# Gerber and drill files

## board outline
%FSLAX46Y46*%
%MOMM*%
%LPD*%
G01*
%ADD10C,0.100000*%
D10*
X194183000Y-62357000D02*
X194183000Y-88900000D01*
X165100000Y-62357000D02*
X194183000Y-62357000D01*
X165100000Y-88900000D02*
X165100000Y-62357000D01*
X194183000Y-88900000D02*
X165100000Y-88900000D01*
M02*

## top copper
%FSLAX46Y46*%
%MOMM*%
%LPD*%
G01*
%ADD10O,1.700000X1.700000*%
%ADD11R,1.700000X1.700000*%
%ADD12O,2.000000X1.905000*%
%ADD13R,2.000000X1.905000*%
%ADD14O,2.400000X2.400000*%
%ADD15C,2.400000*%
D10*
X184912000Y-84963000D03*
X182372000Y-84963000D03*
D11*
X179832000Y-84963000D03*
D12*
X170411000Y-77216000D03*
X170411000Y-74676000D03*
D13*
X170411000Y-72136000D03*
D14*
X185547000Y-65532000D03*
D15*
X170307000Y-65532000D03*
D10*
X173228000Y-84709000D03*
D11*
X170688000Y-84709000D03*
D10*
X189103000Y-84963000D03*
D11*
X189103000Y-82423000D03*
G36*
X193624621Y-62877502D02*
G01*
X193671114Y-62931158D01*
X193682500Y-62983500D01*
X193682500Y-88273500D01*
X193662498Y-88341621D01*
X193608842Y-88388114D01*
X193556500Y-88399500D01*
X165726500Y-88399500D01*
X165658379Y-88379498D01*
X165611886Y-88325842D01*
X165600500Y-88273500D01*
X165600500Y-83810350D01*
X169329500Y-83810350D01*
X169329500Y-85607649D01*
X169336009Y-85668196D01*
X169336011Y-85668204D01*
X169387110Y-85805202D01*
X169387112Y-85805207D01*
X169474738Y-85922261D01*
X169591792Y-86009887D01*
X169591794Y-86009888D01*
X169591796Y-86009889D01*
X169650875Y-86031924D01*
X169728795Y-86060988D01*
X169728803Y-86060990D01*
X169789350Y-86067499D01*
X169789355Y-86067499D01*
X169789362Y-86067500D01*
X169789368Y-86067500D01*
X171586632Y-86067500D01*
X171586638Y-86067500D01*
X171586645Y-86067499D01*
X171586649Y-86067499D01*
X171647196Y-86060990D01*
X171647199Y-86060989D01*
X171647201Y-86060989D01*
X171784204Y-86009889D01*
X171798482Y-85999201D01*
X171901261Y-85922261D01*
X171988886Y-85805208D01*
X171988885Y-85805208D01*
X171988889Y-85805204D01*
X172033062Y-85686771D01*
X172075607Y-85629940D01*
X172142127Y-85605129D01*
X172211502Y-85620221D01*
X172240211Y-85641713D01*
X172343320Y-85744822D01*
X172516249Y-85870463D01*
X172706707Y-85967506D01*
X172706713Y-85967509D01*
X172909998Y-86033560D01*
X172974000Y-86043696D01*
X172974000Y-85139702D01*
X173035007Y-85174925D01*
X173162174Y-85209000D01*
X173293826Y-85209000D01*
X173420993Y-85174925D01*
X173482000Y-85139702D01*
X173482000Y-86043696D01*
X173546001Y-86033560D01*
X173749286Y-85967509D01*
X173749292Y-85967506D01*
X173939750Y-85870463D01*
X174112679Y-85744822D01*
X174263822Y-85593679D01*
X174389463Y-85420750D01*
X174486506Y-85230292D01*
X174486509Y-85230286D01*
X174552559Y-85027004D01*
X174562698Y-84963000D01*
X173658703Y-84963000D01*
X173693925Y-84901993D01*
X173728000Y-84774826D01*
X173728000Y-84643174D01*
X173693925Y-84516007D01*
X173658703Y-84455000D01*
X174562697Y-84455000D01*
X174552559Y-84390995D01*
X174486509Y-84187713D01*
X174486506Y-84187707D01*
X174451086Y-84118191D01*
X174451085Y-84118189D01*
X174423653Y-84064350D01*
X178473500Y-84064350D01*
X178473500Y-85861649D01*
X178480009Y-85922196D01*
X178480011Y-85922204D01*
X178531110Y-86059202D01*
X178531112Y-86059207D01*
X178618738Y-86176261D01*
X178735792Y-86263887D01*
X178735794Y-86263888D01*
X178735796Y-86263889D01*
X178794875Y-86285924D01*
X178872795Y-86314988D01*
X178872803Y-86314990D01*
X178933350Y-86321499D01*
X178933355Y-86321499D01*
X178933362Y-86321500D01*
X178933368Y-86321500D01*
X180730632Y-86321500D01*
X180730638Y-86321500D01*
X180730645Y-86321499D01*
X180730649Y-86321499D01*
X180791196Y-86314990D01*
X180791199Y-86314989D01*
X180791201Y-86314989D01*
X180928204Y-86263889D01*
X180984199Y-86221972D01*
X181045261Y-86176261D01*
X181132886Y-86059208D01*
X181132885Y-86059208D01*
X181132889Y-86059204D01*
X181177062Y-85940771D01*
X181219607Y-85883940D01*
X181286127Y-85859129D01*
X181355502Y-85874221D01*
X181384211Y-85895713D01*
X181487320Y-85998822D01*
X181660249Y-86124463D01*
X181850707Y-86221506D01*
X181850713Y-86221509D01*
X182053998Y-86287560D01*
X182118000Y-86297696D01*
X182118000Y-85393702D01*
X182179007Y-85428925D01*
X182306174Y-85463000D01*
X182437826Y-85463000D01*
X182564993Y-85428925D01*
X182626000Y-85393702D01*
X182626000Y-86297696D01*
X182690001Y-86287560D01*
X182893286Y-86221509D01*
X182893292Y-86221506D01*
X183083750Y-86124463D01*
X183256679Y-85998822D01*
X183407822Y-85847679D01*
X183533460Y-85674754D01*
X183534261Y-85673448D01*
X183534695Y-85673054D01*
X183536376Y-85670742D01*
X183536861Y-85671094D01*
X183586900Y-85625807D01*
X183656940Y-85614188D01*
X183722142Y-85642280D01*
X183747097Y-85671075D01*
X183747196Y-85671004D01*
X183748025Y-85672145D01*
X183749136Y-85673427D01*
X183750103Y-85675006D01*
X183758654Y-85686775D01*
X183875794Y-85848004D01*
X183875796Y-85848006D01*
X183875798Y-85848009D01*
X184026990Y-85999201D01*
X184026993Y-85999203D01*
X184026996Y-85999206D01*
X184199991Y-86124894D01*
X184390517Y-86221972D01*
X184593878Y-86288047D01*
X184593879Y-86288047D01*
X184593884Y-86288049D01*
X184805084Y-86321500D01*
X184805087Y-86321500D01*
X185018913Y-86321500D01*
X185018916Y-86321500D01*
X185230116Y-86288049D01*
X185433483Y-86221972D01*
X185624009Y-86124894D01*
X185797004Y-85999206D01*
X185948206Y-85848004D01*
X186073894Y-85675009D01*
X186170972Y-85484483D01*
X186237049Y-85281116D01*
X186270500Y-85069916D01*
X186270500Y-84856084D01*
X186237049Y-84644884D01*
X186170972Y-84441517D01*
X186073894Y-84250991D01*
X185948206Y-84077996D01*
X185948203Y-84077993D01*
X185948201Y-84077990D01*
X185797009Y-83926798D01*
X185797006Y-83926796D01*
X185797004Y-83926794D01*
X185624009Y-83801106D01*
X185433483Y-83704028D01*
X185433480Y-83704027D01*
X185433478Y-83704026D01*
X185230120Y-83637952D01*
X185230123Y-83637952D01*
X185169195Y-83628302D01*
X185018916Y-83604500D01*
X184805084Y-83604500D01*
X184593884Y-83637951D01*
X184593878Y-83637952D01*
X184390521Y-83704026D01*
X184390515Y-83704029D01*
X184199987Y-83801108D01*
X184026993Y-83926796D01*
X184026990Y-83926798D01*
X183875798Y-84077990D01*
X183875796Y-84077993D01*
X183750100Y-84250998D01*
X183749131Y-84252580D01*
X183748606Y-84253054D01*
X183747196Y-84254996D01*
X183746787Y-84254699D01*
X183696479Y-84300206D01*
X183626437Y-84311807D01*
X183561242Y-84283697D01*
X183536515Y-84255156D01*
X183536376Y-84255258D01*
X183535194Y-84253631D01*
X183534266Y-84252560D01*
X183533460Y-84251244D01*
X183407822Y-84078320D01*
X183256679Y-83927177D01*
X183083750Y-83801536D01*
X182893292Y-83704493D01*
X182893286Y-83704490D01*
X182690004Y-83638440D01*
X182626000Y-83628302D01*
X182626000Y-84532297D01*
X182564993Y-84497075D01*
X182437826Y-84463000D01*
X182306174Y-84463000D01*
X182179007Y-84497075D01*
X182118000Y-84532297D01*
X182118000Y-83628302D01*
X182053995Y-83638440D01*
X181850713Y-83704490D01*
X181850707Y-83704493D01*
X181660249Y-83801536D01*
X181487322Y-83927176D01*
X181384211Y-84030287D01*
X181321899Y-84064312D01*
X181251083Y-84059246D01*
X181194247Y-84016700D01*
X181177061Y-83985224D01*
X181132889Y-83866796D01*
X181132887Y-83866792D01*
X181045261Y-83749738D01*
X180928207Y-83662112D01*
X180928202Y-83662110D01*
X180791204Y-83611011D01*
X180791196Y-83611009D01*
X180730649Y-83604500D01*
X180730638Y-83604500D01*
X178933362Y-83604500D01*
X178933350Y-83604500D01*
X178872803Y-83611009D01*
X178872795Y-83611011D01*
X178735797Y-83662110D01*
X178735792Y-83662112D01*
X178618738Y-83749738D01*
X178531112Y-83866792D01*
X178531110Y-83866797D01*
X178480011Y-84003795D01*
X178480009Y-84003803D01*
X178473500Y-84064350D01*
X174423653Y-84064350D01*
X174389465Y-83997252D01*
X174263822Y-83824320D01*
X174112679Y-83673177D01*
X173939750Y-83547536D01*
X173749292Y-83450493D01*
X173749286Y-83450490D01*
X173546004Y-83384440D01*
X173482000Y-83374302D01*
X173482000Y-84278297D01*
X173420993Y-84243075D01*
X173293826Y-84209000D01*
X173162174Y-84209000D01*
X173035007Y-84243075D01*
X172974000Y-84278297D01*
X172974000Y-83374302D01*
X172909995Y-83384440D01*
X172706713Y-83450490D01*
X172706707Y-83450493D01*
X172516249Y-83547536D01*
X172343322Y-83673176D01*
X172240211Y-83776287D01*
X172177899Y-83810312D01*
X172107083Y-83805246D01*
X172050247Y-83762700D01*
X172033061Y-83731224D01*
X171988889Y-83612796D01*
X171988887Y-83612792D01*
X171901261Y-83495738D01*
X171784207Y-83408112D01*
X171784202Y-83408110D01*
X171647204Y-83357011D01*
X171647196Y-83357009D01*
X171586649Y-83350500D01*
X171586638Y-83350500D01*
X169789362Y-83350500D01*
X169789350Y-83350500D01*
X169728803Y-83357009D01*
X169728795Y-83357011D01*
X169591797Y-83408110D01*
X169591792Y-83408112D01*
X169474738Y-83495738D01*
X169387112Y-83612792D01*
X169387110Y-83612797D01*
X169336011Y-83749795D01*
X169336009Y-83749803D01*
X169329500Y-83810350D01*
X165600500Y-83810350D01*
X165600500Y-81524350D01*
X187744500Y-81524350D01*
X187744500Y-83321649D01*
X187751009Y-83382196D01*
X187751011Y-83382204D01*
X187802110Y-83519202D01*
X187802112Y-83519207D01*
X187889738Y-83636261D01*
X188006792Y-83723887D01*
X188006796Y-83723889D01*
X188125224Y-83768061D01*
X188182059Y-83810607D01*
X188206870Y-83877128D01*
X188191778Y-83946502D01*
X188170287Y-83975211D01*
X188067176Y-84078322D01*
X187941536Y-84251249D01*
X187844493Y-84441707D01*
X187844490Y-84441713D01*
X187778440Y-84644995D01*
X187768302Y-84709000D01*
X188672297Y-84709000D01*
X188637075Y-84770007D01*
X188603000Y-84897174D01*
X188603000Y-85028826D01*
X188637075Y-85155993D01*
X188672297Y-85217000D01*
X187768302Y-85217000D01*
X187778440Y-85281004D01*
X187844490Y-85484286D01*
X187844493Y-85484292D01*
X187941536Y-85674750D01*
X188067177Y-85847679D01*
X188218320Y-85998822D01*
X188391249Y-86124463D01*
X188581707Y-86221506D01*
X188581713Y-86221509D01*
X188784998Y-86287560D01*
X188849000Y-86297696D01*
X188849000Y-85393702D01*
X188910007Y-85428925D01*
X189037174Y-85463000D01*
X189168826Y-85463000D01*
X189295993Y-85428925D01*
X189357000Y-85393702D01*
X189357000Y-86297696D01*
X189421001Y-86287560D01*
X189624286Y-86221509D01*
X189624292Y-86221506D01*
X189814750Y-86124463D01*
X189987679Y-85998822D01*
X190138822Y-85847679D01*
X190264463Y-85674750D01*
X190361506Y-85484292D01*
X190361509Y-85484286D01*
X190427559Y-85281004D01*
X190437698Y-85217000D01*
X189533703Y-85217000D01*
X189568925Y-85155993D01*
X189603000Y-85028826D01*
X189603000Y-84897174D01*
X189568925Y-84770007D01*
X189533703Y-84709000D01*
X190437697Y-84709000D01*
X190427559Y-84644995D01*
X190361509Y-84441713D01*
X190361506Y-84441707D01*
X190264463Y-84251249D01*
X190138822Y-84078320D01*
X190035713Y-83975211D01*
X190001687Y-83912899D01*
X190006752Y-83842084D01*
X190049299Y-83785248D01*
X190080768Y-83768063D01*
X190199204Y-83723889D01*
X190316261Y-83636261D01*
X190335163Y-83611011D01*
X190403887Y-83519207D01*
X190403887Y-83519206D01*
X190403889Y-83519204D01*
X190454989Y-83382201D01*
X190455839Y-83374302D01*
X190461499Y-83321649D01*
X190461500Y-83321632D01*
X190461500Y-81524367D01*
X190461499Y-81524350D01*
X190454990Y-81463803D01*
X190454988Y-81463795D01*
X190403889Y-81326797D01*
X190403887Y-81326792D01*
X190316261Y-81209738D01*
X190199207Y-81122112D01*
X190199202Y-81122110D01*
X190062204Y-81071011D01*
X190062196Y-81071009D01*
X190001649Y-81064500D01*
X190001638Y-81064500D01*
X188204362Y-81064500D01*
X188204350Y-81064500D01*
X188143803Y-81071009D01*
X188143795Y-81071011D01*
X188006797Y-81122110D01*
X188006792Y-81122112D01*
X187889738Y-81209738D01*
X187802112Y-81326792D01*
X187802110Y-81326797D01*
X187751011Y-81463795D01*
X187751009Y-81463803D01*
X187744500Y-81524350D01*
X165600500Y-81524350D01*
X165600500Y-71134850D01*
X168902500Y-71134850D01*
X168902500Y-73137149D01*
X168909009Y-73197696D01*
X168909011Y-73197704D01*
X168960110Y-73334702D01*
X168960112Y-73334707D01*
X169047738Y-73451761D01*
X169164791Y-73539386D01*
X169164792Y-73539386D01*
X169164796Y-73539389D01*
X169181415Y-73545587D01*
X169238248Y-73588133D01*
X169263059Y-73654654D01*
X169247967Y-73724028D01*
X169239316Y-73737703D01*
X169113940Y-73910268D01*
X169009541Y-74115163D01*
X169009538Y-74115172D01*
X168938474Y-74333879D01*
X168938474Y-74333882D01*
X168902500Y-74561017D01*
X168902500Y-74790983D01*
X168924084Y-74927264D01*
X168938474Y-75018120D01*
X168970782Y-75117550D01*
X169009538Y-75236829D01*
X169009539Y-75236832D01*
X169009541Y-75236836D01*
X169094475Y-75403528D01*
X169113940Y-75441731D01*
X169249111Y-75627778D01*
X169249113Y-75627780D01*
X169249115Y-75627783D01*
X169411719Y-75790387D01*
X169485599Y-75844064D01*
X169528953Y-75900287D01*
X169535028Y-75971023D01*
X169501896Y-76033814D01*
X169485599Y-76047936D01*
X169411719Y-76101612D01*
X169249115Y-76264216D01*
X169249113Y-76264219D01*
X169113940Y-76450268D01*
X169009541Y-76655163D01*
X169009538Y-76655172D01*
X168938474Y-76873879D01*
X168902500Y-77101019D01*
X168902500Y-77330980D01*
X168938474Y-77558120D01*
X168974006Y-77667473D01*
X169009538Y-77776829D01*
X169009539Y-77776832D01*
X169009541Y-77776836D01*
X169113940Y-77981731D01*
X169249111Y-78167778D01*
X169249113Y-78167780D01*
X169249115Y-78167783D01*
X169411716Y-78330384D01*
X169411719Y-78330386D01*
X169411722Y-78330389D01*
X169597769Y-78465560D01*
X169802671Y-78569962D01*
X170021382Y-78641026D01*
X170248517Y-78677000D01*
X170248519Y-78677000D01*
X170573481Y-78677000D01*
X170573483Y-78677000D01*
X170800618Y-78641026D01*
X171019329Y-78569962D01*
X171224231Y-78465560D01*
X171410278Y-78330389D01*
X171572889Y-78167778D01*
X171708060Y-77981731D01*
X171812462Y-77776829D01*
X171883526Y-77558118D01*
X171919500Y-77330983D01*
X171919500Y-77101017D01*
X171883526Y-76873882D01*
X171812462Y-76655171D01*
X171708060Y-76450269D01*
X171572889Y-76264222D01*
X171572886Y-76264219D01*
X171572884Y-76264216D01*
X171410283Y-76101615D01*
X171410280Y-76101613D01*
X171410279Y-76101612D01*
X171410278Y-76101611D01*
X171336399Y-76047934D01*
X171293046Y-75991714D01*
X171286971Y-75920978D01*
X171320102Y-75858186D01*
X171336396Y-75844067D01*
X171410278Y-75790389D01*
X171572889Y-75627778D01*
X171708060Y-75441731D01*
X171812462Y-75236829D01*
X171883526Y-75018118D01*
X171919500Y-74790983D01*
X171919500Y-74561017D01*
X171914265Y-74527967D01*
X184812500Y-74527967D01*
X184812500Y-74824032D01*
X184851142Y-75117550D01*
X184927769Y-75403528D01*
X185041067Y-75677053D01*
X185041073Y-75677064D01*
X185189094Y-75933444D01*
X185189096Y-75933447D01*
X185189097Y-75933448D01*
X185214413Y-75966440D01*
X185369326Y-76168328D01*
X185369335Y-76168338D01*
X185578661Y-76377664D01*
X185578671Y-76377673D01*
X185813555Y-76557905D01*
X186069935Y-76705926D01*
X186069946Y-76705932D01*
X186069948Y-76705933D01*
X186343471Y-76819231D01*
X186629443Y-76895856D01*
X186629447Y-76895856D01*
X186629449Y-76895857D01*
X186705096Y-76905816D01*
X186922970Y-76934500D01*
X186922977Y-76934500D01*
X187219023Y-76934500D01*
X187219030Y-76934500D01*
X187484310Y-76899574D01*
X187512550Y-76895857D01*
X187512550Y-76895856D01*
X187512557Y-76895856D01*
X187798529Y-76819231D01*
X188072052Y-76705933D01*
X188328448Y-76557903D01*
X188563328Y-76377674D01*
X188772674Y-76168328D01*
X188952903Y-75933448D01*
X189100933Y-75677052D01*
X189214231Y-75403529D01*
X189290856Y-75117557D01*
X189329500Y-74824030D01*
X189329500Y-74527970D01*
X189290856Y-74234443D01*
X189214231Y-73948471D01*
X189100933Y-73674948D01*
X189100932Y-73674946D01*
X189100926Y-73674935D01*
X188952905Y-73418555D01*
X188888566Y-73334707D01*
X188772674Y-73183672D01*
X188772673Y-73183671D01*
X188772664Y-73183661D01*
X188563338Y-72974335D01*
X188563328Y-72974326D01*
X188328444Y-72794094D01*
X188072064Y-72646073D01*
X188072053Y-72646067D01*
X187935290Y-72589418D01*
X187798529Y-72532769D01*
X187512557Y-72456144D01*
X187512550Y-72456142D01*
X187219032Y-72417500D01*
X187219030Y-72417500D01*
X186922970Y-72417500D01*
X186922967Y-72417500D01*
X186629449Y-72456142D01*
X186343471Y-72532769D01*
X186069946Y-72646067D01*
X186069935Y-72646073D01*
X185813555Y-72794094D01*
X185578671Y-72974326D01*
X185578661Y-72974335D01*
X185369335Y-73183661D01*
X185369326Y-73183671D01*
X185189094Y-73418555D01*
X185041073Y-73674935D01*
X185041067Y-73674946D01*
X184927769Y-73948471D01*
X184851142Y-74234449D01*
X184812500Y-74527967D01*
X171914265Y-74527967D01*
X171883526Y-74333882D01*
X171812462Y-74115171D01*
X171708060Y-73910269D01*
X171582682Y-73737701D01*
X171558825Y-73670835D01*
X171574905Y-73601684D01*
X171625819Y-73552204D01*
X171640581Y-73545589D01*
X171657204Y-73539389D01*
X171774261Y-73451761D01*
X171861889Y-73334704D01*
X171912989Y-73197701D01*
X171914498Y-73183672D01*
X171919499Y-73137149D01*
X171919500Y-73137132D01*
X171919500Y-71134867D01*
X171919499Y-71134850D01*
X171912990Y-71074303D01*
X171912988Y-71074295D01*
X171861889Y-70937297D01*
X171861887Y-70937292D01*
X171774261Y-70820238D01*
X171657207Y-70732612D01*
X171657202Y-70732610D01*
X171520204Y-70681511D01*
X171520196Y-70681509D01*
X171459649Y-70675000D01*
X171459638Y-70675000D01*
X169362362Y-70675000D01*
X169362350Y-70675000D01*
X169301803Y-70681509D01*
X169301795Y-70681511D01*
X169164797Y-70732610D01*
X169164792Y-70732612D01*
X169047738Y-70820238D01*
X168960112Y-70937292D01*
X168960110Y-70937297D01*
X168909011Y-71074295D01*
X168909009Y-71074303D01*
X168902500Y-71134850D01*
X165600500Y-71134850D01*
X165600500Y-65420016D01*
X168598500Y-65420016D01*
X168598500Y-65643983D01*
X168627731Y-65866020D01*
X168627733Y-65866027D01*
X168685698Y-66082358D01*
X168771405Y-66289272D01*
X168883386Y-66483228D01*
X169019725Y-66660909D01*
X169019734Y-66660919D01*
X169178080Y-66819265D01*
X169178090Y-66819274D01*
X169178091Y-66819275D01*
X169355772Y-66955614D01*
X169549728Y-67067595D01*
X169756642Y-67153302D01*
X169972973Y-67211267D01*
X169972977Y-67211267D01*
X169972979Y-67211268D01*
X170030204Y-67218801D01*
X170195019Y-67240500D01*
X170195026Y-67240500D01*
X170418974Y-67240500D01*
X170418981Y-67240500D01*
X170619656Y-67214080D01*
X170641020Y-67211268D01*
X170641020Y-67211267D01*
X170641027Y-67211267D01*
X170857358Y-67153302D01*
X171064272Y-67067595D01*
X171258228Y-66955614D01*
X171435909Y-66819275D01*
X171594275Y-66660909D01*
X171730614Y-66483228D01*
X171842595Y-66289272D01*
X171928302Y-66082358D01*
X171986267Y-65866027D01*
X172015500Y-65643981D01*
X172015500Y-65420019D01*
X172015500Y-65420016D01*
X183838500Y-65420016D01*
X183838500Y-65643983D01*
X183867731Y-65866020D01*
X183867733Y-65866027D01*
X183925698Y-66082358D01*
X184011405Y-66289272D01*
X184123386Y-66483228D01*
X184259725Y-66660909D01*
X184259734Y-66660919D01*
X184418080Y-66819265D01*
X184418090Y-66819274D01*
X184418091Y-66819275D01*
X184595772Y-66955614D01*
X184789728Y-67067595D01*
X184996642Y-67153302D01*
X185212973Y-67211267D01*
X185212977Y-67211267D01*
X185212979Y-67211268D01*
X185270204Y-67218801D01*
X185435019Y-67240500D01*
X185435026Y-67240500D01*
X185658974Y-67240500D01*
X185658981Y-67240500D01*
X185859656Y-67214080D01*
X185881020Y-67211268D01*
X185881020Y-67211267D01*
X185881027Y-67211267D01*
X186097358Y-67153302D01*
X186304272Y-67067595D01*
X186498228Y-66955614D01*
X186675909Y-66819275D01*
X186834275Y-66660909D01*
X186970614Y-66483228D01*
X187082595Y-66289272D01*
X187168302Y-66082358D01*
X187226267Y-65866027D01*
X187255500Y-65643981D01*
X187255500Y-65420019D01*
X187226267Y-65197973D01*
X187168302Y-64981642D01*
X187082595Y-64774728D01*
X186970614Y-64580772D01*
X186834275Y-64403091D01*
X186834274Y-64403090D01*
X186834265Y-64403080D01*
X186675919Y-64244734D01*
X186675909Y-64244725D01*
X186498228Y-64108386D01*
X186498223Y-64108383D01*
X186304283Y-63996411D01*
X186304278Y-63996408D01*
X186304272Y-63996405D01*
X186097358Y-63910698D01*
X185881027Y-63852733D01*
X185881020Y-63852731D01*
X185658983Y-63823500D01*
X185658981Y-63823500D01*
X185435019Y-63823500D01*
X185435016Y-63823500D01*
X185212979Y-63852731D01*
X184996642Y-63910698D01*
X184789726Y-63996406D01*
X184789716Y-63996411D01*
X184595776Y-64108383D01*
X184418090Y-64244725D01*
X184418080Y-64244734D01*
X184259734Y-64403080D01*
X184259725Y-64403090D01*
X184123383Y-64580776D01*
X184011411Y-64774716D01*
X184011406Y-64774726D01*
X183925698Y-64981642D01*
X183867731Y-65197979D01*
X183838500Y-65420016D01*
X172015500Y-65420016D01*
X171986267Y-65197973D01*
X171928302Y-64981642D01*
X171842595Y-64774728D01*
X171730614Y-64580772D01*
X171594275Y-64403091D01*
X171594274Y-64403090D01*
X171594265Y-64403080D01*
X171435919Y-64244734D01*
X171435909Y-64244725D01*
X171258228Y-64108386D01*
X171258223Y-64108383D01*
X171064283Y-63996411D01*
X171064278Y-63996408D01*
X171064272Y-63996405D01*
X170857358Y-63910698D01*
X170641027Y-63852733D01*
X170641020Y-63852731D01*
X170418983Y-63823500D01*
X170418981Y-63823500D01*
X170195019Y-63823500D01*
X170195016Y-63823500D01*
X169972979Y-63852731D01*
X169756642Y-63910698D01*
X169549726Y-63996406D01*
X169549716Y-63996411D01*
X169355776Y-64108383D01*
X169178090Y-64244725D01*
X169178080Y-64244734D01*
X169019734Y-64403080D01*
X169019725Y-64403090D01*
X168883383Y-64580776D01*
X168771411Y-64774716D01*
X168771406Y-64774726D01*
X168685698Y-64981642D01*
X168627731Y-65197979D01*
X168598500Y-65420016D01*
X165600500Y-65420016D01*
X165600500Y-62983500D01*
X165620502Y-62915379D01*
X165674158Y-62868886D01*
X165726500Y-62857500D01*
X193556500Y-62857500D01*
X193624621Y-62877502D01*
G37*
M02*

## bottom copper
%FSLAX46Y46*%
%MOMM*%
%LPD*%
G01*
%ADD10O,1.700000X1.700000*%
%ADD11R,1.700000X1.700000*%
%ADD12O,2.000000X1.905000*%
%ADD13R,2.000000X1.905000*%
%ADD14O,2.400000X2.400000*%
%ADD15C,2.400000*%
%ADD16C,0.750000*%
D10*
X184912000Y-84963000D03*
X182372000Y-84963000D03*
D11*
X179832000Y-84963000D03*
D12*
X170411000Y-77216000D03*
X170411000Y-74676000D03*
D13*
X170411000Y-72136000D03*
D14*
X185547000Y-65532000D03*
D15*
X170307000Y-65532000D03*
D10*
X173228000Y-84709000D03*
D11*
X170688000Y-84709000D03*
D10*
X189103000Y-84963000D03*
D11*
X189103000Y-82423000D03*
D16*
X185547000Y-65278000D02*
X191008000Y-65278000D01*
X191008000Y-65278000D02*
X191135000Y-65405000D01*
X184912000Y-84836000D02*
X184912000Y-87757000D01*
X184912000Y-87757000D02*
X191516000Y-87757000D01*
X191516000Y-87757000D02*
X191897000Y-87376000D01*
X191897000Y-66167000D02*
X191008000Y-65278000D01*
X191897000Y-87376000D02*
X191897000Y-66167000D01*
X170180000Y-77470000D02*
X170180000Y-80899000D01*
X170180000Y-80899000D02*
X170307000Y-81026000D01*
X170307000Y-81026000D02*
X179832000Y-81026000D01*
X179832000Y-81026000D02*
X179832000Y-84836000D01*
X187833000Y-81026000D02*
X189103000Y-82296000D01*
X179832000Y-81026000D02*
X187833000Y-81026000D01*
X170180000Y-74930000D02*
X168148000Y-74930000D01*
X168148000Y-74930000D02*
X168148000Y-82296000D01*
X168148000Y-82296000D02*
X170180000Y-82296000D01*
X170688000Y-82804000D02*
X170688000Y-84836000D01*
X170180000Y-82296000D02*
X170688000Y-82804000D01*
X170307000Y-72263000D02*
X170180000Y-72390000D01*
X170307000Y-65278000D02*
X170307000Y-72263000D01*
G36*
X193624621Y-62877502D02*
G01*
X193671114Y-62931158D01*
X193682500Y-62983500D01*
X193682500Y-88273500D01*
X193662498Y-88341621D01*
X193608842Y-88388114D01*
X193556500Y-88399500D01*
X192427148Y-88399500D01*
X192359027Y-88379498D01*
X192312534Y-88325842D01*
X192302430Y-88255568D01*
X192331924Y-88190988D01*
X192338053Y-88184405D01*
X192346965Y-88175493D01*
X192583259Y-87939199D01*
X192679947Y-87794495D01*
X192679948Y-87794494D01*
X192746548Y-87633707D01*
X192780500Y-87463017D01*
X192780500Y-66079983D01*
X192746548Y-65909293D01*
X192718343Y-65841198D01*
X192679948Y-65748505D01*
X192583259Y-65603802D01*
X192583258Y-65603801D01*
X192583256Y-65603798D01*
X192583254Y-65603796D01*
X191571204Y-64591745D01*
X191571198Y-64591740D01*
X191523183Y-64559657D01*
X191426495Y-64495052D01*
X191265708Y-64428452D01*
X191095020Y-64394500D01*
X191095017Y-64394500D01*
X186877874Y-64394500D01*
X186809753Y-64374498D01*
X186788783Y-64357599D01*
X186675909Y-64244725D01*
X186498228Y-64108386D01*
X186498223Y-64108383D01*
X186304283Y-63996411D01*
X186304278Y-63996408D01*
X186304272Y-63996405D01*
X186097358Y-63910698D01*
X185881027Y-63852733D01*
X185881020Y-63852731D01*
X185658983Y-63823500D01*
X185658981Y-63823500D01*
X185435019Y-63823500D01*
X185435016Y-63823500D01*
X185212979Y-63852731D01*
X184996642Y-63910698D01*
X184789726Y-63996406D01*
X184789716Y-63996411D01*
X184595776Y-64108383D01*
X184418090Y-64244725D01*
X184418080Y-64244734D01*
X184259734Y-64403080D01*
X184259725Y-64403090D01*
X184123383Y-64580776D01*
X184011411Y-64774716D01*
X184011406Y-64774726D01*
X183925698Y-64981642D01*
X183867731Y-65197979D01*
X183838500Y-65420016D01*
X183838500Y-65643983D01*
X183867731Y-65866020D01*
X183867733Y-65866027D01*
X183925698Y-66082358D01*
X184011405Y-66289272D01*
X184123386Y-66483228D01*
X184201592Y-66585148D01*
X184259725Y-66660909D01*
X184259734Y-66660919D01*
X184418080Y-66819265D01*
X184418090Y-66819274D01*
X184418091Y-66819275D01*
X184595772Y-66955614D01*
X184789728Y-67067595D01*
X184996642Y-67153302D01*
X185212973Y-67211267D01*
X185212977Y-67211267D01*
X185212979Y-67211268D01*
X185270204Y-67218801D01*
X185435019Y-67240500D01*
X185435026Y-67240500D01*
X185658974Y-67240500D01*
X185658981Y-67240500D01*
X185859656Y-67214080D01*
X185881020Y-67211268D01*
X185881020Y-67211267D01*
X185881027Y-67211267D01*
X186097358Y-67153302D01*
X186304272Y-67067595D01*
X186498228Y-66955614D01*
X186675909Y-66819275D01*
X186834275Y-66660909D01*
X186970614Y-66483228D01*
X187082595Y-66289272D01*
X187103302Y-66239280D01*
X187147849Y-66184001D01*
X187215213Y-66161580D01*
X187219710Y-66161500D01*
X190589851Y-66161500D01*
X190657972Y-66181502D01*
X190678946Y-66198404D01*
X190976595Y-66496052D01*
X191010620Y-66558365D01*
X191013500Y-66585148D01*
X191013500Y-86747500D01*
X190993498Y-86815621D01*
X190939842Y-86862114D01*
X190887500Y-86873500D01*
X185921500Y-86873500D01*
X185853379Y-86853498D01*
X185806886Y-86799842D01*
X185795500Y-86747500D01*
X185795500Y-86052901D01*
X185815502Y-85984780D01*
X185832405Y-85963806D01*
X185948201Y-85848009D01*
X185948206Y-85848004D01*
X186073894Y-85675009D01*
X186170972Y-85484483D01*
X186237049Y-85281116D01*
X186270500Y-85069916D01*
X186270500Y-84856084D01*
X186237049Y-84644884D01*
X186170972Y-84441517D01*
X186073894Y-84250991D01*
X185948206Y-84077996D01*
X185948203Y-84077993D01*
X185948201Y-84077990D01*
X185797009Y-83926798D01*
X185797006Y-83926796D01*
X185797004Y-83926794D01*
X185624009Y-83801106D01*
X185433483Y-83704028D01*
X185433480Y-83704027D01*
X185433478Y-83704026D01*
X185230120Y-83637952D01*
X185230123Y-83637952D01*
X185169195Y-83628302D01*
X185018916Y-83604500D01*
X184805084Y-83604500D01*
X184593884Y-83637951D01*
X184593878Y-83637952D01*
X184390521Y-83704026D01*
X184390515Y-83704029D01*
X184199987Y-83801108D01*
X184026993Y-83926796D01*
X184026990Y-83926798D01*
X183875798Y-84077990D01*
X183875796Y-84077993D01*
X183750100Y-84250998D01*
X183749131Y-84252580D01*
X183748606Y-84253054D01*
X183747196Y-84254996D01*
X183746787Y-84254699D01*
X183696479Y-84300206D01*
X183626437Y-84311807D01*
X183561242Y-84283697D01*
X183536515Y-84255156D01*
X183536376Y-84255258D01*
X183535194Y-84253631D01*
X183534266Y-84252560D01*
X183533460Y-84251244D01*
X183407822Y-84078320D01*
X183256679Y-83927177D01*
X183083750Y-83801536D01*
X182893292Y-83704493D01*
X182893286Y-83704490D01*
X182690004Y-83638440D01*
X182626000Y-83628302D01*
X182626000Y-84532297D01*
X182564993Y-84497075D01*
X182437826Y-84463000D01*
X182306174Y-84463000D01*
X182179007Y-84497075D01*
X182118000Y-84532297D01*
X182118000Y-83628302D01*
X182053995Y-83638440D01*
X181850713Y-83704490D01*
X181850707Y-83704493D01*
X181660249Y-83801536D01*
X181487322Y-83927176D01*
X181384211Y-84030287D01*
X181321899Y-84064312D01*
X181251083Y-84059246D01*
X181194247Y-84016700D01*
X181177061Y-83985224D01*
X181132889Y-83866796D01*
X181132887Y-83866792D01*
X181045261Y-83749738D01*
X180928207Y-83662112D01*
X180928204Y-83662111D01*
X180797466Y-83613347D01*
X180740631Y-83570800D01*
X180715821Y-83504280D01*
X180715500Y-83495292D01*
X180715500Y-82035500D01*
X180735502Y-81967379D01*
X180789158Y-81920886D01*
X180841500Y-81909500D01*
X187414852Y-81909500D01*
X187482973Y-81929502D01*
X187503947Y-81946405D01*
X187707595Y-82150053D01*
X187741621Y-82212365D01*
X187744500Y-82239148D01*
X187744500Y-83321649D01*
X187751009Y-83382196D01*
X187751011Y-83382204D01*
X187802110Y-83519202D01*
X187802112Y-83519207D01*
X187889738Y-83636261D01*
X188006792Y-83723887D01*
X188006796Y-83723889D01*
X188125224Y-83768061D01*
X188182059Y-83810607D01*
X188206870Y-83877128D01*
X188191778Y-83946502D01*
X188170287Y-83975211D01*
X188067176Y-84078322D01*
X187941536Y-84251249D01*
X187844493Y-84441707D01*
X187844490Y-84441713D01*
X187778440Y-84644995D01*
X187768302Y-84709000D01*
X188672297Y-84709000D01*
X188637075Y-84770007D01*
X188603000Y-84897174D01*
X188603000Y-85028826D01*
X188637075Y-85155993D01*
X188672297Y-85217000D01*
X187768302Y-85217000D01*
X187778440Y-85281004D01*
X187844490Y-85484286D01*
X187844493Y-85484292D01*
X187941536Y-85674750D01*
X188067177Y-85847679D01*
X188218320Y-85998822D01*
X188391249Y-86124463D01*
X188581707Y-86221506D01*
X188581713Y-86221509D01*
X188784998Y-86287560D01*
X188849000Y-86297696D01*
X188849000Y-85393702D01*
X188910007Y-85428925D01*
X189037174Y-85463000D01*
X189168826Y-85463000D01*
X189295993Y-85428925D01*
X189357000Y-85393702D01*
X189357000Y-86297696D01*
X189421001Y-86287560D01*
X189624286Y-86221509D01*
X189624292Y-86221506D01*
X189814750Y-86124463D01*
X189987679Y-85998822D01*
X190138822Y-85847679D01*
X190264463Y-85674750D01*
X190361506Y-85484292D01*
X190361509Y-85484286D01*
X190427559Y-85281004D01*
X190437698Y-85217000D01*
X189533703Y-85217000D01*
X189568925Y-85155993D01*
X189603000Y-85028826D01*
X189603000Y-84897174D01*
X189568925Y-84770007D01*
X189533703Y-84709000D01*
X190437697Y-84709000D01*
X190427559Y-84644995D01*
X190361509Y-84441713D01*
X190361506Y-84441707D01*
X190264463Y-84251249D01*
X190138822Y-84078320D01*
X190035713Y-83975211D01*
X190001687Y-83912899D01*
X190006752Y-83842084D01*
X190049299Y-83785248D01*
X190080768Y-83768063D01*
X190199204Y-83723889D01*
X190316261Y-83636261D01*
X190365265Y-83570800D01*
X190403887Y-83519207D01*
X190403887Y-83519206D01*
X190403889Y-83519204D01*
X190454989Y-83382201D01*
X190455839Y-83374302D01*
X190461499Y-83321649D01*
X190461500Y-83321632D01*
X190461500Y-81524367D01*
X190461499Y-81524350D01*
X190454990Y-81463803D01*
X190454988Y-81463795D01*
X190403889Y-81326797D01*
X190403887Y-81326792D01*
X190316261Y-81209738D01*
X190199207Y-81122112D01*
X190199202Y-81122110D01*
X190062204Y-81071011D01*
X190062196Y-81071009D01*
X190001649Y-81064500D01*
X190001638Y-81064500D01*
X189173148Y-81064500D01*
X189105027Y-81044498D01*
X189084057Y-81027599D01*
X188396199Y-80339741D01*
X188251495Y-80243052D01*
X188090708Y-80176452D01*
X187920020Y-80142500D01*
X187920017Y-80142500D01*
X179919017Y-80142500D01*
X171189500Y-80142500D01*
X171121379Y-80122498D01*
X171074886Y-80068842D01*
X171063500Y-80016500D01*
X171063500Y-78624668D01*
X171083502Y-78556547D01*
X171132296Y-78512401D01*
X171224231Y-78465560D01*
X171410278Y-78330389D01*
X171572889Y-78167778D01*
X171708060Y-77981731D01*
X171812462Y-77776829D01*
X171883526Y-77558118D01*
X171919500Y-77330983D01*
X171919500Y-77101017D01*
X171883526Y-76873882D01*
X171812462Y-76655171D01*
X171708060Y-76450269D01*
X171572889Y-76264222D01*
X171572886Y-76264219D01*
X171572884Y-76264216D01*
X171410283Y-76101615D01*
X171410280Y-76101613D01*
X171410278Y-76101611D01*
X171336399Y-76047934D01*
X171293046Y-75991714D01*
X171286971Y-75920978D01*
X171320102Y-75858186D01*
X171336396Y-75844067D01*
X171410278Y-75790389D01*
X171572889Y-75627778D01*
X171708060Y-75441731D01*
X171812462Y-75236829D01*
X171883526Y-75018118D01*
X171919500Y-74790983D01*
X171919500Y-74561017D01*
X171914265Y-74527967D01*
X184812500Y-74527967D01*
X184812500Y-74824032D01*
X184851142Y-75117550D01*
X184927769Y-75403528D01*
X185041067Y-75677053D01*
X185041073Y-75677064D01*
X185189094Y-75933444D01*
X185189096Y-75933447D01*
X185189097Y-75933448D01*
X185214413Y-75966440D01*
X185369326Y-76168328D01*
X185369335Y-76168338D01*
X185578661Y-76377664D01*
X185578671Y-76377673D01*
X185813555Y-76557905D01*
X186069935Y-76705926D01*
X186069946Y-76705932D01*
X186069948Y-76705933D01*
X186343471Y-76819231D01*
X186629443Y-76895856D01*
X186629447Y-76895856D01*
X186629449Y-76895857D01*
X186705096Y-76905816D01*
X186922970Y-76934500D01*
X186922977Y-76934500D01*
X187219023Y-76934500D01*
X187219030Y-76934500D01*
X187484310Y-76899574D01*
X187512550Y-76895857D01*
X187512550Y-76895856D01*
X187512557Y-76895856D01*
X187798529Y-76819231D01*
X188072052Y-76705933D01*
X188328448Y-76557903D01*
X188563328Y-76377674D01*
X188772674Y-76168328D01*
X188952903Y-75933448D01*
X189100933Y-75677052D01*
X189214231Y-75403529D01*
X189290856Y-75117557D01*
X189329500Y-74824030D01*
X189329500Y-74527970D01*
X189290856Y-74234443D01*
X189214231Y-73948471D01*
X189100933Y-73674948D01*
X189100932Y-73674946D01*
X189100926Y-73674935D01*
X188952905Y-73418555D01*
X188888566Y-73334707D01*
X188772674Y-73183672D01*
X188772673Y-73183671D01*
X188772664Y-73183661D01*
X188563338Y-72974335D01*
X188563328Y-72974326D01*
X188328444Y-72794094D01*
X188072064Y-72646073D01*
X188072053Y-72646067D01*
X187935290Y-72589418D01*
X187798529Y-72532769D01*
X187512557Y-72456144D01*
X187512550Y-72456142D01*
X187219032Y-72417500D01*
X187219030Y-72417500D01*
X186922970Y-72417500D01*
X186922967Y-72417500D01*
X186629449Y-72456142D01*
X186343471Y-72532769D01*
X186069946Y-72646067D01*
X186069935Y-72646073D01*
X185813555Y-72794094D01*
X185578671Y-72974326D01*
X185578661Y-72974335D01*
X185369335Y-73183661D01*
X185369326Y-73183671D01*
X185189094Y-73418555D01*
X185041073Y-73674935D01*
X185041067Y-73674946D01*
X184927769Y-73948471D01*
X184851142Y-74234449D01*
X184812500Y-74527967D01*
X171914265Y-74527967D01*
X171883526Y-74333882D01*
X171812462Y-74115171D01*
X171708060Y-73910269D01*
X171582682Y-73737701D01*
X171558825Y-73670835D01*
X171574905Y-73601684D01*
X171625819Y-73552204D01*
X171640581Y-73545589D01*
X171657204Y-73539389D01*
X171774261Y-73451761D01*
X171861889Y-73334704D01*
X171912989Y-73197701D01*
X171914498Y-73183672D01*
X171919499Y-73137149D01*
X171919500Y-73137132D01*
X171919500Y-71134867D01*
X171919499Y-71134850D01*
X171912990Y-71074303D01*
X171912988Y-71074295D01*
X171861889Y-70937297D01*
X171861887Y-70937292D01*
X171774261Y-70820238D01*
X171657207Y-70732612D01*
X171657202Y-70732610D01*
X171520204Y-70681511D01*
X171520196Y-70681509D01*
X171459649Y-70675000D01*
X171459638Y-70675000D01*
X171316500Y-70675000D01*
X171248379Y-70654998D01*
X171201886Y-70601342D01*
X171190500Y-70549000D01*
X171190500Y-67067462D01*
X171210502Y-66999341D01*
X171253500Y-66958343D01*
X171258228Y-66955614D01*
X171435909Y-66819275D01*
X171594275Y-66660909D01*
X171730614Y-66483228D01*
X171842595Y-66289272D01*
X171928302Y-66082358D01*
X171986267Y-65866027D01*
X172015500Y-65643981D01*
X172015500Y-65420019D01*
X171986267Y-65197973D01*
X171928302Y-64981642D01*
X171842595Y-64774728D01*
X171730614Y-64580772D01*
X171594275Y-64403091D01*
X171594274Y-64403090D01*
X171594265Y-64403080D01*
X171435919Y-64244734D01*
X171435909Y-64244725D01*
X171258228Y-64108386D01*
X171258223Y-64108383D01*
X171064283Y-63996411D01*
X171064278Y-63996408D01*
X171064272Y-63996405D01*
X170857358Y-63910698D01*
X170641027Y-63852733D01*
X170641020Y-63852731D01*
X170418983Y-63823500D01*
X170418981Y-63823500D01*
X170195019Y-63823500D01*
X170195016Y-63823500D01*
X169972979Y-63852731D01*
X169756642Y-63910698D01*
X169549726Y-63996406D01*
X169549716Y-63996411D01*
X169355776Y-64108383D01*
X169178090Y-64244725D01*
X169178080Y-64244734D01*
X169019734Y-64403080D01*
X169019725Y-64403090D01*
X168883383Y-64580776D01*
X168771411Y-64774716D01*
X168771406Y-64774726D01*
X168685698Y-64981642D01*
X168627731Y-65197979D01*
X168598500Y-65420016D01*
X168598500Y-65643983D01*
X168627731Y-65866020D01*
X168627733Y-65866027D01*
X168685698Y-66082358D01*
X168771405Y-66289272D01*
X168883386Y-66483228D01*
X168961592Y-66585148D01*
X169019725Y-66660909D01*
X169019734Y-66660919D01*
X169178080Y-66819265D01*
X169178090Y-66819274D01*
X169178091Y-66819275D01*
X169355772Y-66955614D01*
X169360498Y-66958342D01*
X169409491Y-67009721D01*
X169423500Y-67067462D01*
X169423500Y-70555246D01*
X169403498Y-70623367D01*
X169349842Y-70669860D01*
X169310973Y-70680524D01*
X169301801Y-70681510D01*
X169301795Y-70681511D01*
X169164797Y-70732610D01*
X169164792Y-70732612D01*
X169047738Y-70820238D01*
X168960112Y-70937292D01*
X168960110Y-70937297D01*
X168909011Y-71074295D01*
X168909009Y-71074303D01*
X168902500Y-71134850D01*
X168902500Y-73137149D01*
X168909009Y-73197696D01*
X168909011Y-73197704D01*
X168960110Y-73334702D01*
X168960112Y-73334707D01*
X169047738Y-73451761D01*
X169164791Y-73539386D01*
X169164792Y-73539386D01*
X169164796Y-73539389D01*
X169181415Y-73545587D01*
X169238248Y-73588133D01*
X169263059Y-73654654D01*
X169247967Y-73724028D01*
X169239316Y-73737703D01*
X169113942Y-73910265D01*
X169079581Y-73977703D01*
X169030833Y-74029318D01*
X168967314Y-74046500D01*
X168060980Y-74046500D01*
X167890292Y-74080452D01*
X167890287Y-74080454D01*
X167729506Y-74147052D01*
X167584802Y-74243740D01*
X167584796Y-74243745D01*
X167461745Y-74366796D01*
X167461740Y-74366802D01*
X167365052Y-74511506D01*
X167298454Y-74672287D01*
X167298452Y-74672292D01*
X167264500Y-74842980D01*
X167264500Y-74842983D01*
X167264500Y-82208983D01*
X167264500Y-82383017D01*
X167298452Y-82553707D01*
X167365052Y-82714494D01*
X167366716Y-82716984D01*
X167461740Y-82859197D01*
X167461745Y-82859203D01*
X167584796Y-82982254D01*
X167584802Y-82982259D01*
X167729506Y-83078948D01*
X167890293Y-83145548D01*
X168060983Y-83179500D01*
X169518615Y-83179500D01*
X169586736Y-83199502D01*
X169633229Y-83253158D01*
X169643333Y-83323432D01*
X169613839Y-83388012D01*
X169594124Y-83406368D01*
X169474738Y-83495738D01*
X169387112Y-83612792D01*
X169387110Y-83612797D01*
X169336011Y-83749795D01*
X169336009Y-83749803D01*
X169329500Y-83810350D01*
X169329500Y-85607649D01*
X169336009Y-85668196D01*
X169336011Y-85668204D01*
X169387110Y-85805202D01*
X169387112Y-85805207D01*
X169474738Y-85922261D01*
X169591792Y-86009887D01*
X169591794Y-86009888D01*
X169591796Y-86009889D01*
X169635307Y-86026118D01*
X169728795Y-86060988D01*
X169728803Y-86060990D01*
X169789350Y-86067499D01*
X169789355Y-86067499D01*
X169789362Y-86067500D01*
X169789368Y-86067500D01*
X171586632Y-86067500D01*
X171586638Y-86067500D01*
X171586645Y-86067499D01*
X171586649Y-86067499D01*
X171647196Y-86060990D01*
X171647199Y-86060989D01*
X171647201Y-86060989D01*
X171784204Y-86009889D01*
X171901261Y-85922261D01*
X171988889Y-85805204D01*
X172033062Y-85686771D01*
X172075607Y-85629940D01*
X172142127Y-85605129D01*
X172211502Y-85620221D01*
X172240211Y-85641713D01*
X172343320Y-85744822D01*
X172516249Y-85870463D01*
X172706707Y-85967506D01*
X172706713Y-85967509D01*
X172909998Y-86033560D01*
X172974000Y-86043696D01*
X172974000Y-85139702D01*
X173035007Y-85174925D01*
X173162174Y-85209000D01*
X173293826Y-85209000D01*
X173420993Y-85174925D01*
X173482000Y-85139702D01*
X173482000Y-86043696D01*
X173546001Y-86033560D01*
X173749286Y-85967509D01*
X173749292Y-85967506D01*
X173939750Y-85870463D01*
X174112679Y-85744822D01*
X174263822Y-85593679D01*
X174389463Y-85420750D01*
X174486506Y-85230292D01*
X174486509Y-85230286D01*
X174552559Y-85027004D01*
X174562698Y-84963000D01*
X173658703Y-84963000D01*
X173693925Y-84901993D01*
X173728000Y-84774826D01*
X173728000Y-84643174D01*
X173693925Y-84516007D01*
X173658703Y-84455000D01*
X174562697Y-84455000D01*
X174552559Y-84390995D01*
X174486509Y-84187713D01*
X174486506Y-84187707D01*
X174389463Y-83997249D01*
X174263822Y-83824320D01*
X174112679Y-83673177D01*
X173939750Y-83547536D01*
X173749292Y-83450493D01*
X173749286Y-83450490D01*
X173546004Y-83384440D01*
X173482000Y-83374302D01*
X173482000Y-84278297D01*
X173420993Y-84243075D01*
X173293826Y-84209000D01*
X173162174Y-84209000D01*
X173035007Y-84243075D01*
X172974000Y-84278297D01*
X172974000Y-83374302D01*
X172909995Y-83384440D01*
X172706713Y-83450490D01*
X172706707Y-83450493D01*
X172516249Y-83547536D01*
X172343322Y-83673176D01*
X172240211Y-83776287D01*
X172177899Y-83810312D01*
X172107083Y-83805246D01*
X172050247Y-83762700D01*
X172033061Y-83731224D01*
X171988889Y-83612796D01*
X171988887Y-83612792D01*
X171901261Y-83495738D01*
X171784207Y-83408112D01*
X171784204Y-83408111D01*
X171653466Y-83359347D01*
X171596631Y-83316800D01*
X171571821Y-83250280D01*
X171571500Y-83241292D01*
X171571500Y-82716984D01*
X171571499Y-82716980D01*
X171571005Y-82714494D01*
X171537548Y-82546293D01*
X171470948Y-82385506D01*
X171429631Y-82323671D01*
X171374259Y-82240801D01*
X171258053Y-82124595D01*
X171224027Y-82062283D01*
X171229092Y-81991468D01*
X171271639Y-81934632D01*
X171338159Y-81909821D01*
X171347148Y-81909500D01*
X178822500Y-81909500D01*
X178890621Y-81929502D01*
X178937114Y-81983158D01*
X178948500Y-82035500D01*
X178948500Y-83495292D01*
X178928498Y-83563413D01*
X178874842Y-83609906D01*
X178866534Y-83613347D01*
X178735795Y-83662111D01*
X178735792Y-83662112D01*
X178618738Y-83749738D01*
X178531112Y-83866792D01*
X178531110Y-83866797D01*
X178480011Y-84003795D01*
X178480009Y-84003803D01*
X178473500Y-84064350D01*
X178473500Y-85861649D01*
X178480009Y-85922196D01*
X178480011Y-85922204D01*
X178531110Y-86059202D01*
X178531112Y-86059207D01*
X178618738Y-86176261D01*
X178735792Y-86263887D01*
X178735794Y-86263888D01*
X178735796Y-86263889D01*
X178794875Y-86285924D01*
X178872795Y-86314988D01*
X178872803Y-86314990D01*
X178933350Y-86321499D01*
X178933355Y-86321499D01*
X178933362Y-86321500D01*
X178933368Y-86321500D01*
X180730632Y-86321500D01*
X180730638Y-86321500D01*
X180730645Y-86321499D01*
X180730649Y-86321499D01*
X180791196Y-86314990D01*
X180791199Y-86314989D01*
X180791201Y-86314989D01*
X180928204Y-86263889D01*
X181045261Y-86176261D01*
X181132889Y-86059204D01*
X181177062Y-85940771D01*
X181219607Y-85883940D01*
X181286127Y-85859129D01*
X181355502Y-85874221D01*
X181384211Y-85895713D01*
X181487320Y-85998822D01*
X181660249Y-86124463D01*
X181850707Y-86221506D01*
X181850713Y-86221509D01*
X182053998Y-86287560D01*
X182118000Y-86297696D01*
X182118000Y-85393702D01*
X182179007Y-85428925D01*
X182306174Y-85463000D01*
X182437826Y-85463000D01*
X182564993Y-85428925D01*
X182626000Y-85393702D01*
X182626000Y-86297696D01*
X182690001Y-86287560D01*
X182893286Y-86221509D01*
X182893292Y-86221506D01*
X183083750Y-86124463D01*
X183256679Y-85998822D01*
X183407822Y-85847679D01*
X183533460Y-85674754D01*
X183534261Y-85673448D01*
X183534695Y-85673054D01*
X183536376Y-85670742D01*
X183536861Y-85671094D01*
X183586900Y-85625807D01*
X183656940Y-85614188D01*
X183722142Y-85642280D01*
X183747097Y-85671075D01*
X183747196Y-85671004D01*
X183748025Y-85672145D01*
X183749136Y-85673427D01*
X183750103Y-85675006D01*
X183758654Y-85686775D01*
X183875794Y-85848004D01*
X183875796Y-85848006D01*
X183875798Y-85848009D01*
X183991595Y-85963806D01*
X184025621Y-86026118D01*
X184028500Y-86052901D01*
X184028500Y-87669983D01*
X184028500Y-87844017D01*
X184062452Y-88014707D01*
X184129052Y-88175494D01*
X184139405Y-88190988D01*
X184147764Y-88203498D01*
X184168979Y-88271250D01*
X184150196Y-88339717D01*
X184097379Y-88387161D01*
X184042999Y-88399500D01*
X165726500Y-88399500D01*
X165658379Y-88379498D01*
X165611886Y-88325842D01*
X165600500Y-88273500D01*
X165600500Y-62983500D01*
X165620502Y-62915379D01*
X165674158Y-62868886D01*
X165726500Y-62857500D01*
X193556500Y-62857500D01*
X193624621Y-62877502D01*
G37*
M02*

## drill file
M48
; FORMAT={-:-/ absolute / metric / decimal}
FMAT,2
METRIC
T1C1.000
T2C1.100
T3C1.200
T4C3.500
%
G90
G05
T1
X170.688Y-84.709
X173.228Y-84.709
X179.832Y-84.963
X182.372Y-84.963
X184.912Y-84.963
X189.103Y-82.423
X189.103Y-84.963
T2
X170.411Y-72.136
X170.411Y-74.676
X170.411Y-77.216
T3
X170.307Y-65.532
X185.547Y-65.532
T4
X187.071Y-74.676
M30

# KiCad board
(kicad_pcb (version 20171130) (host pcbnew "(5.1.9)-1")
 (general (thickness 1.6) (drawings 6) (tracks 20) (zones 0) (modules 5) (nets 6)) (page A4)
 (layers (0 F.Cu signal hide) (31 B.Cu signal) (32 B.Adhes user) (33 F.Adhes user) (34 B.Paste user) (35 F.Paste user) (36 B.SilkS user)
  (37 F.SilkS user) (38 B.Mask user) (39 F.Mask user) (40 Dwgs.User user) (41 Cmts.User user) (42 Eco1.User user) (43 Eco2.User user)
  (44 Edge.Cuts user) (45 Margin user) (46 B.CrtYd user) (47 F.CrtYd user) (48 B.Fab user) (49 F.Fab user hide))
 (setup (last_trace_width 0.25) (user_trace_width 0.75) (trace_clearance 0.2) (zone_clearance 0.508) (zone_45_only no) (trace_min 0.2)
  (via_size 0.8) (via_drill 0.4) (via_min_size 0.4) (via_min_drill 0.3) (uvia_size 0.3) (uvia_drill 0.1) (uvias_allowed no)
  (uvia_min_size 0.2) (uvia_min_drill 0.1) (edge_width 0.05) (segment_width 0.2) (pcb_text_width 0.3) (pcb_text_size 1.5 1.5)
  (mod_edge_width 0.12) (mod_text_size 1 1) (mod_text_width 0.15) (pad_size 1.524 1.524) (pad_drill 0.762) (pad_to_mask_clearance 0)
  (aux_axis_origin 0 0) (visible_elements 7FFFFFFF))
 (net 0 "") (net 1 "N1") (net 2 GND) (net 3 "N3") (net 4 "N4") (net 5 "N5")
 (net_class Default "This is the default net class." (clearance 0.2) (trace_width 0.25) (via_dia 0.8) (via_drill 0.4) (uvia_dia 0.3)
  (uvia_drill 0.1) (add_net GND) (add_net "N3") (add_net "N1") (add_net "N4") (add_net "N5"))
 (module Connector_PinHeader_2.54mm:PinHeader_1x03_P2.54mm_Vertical (layer F.Cu) (at 179.832 84.963 90)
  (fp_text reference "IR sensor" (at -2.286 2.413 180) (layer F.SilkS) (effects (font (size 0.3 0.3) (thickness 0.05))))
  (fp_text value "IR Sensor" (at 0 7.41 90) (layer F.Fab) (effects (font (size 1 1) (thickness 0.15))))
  (pad 3 thru_hole oval (at 0 5.08 90) (size 1.7 1.7) (drill 1) (layers *.Cu *.Mask) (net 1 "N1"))
  (pad 2 thru_hole oval (at 0 2.54 90) (size 1.7 1.7) (drill 1) (layers *.Cu *.Mask) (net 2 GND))
  (pad 1 thru_hole rect (at 0 0 90) (size 1.7 1.7) (drill 1) (layers *.Cu *.Mask) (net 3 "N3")))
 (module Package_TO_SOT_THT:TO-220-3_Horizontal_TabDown (layer F.Cu) (at 170.411 72.136 270)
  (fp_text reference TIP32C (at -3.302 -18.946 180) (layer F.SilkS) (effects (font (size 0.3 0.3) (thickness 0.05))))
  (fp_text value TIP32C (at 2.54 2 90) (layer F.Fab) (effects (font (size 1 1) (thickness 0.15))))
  (pad 3 thru_hole oval (at 5.08 0 270) (size 1.905 2) (drill 1.1) (layers *.Cu *.Mask) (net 3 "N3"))
  (pad 2 thru_hole oval (at 2.54 0 270) (size 1.905 2) (drill 1.1) (layers *.Cu *.Mask) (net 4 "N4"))
  (pad 1 thru_hole rect (at 0 0 270) (size 1.905 2) (drill 1.1) (layers *.Cu *.Mask) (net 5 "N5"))
  (pad "" np_thru_hole oval (at 2.54 -16.66 270) (size 3.5 3.5) (drill 3.5) (layers *.Cu *.Mask)))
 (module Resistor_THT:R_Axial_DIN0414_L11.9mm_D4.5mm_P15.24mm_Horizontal (layer F.Cu) (at 170.307 65.532)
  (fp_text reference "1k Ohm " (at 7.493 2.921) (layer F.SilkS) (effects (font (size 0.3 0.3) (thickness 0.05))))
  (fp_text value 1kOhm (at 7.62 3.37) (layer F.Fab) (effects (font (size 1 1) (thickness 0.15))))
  (pad 2 thru_hole oval (at 15.24 0) (size 2.4 2.4) (drill 1.2) (layers *.Cu *.Mask) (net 1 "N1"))
  (pad 1 thru_hole circle (at 0 0) (size 2.4 2.4) (drill 1.2) (layers *.Cu *.Mask) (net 5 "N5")))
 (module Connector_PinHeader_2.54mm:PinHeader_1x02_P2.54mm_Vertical (layer F.Cu) (at 170.688 84.709 90)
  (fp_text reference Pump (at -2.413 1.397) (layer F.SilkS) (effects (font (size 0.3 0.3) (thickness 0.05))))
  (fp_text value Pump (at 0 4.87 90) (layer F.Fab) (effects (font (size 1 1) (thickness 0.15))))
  (pad 2 thru_hole oval (at 0 2.54 90) (size 1.7 1.7) (drill 1) (layers *.Cu *.Mask) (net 2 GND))
  (pad 1 thru_hole rect (at 0 0 90) (size 1.7 1.7) (drill 1) (layers *.Cu *.Mask) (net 4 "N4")))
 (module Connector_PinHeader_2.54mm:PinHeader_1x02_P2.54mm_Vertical (layer F.Cu) (at 189.103 82.423)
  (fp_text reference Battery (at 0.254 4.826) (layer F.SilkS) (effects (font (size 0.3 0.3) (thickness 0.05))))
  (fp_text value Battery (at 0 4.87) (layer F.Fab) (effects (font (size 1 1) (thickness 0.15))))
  (pad 2 thru_hole oval (at 0 2.54) (size 1.7 1.7) (drill 1) (layers *.Cu *.Mask) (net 2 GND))
  (pad 1 thru_hole rect (at 0 0) (size 1.7 1.7) (drill 1) (layers *.Cu *.Mask) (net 3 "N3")))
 (gr_line (start 194.183 62.357) (end 194.183 88.9) (layer Edge.Cuts) (width 0.1))
 (gr_line (start 165.1 62.357) (end 194.183 62.357) (layer Edge.Cuts) (width 0.1))
 (gr_line (start 165.1 88.9) (end 165.1 62.357) (layer Edge.Cuts) (width 0.1))
 (gr_line (start 194.183 88.9) (end 165.1 88.9) (layer Edge.Cuts) (width 0.1))
 (segment (start 185.547 65.278) (end 191.008 65.278) (width 0.75) (layer B.Cu) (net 1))
 (segment (start 191.008 65.278) (end 191.135 65.405) (width 0.75) (layer B.Cu) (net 1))
 (segment (start 184.912 84.836) (end 184.912 87.757) (width 0.75) (layer B.Cu) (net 1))
 (segment (start 184.912 87.757) (end 191.516 87.757) (width 0.75) (layer B.Cu) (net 1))
 (segment (start 191.516 87.757) (end 191.897 87.376) (width 0.75) (layer B.Cu) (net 1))
 (segment (start 191.897 66.167) (end 191.008 65.278) (width 0.75) (layer B.Cu) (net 1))
 (segment (start 191.897 87.376) (end 191.897 66.167) (width 0.75) (layer B.Cu) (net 1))
 (segment (start 170.18 77.47) (end 170.18 80.899) (width 0.75) (layer B.Cu) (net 3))
 (segment (start 170.18 80.899) (end 170.307 81.026) (width 0.75) (layer B.Cu) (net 3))
 (segment (start 170.307 81.026) (end 179.832 81.026) (width 0.75) (layer B.Cu) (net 3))
 (segment (start 179.832 81.026) (end 179.832 84.836) (width 0.75) (layer B.Cu) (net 3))
 (segment (start 187.833 81.026) (end 189.103 82.296) (width 0.75) (layer B.Cu) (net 3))
 (segment (start 179.832 81.026) (end 187.833 81.026) (width 0.75) (layer B.Cu) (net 3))
 (segment (start 170.18 74.93) (end 168.148 74.93) (width 0.75) (layer B.Cu) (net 4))
 (segment (start 168.148 74.93) (end 168.148 82.296) (width 0.75) (layer B.Cu) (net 4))
 (segment (start 168.148 82.296) (end 170.18 82.296) (width 0.75) (layer B.Cu) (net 4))
 (segment (start 170.688 82.804) (end 170.688 84.836) (width 0.75) (layer B.Cu) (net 4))
 (segment (start 170.18 82.296) (end 170.688 82.804) (width 0.75) (layer B.Cu) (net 4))
 (segment (start 170.307 72.263) (end 170.18 72.39) (width 0.75) (layer B.Cu) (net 5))
 (segment (start 170.307 65.278) (end 170.307 72.263) (width 0.75) (layer B.Cu) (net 5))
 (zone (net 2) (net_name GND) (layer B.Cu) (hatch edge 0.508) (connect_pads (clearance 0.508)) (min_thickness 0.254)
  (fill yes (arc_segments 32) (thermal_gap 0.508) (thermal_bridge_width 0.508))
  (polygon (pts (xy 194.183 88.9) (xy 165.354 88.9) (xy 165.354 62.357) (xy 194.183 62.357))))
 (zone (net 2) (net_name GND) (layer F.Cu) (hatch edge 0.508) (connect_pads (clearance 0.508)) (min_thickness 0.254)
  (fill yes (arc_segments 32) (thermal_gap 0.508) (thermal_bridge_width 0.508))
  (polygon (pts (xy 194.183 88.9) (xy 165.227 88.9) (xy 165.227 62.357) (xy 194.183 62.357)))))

